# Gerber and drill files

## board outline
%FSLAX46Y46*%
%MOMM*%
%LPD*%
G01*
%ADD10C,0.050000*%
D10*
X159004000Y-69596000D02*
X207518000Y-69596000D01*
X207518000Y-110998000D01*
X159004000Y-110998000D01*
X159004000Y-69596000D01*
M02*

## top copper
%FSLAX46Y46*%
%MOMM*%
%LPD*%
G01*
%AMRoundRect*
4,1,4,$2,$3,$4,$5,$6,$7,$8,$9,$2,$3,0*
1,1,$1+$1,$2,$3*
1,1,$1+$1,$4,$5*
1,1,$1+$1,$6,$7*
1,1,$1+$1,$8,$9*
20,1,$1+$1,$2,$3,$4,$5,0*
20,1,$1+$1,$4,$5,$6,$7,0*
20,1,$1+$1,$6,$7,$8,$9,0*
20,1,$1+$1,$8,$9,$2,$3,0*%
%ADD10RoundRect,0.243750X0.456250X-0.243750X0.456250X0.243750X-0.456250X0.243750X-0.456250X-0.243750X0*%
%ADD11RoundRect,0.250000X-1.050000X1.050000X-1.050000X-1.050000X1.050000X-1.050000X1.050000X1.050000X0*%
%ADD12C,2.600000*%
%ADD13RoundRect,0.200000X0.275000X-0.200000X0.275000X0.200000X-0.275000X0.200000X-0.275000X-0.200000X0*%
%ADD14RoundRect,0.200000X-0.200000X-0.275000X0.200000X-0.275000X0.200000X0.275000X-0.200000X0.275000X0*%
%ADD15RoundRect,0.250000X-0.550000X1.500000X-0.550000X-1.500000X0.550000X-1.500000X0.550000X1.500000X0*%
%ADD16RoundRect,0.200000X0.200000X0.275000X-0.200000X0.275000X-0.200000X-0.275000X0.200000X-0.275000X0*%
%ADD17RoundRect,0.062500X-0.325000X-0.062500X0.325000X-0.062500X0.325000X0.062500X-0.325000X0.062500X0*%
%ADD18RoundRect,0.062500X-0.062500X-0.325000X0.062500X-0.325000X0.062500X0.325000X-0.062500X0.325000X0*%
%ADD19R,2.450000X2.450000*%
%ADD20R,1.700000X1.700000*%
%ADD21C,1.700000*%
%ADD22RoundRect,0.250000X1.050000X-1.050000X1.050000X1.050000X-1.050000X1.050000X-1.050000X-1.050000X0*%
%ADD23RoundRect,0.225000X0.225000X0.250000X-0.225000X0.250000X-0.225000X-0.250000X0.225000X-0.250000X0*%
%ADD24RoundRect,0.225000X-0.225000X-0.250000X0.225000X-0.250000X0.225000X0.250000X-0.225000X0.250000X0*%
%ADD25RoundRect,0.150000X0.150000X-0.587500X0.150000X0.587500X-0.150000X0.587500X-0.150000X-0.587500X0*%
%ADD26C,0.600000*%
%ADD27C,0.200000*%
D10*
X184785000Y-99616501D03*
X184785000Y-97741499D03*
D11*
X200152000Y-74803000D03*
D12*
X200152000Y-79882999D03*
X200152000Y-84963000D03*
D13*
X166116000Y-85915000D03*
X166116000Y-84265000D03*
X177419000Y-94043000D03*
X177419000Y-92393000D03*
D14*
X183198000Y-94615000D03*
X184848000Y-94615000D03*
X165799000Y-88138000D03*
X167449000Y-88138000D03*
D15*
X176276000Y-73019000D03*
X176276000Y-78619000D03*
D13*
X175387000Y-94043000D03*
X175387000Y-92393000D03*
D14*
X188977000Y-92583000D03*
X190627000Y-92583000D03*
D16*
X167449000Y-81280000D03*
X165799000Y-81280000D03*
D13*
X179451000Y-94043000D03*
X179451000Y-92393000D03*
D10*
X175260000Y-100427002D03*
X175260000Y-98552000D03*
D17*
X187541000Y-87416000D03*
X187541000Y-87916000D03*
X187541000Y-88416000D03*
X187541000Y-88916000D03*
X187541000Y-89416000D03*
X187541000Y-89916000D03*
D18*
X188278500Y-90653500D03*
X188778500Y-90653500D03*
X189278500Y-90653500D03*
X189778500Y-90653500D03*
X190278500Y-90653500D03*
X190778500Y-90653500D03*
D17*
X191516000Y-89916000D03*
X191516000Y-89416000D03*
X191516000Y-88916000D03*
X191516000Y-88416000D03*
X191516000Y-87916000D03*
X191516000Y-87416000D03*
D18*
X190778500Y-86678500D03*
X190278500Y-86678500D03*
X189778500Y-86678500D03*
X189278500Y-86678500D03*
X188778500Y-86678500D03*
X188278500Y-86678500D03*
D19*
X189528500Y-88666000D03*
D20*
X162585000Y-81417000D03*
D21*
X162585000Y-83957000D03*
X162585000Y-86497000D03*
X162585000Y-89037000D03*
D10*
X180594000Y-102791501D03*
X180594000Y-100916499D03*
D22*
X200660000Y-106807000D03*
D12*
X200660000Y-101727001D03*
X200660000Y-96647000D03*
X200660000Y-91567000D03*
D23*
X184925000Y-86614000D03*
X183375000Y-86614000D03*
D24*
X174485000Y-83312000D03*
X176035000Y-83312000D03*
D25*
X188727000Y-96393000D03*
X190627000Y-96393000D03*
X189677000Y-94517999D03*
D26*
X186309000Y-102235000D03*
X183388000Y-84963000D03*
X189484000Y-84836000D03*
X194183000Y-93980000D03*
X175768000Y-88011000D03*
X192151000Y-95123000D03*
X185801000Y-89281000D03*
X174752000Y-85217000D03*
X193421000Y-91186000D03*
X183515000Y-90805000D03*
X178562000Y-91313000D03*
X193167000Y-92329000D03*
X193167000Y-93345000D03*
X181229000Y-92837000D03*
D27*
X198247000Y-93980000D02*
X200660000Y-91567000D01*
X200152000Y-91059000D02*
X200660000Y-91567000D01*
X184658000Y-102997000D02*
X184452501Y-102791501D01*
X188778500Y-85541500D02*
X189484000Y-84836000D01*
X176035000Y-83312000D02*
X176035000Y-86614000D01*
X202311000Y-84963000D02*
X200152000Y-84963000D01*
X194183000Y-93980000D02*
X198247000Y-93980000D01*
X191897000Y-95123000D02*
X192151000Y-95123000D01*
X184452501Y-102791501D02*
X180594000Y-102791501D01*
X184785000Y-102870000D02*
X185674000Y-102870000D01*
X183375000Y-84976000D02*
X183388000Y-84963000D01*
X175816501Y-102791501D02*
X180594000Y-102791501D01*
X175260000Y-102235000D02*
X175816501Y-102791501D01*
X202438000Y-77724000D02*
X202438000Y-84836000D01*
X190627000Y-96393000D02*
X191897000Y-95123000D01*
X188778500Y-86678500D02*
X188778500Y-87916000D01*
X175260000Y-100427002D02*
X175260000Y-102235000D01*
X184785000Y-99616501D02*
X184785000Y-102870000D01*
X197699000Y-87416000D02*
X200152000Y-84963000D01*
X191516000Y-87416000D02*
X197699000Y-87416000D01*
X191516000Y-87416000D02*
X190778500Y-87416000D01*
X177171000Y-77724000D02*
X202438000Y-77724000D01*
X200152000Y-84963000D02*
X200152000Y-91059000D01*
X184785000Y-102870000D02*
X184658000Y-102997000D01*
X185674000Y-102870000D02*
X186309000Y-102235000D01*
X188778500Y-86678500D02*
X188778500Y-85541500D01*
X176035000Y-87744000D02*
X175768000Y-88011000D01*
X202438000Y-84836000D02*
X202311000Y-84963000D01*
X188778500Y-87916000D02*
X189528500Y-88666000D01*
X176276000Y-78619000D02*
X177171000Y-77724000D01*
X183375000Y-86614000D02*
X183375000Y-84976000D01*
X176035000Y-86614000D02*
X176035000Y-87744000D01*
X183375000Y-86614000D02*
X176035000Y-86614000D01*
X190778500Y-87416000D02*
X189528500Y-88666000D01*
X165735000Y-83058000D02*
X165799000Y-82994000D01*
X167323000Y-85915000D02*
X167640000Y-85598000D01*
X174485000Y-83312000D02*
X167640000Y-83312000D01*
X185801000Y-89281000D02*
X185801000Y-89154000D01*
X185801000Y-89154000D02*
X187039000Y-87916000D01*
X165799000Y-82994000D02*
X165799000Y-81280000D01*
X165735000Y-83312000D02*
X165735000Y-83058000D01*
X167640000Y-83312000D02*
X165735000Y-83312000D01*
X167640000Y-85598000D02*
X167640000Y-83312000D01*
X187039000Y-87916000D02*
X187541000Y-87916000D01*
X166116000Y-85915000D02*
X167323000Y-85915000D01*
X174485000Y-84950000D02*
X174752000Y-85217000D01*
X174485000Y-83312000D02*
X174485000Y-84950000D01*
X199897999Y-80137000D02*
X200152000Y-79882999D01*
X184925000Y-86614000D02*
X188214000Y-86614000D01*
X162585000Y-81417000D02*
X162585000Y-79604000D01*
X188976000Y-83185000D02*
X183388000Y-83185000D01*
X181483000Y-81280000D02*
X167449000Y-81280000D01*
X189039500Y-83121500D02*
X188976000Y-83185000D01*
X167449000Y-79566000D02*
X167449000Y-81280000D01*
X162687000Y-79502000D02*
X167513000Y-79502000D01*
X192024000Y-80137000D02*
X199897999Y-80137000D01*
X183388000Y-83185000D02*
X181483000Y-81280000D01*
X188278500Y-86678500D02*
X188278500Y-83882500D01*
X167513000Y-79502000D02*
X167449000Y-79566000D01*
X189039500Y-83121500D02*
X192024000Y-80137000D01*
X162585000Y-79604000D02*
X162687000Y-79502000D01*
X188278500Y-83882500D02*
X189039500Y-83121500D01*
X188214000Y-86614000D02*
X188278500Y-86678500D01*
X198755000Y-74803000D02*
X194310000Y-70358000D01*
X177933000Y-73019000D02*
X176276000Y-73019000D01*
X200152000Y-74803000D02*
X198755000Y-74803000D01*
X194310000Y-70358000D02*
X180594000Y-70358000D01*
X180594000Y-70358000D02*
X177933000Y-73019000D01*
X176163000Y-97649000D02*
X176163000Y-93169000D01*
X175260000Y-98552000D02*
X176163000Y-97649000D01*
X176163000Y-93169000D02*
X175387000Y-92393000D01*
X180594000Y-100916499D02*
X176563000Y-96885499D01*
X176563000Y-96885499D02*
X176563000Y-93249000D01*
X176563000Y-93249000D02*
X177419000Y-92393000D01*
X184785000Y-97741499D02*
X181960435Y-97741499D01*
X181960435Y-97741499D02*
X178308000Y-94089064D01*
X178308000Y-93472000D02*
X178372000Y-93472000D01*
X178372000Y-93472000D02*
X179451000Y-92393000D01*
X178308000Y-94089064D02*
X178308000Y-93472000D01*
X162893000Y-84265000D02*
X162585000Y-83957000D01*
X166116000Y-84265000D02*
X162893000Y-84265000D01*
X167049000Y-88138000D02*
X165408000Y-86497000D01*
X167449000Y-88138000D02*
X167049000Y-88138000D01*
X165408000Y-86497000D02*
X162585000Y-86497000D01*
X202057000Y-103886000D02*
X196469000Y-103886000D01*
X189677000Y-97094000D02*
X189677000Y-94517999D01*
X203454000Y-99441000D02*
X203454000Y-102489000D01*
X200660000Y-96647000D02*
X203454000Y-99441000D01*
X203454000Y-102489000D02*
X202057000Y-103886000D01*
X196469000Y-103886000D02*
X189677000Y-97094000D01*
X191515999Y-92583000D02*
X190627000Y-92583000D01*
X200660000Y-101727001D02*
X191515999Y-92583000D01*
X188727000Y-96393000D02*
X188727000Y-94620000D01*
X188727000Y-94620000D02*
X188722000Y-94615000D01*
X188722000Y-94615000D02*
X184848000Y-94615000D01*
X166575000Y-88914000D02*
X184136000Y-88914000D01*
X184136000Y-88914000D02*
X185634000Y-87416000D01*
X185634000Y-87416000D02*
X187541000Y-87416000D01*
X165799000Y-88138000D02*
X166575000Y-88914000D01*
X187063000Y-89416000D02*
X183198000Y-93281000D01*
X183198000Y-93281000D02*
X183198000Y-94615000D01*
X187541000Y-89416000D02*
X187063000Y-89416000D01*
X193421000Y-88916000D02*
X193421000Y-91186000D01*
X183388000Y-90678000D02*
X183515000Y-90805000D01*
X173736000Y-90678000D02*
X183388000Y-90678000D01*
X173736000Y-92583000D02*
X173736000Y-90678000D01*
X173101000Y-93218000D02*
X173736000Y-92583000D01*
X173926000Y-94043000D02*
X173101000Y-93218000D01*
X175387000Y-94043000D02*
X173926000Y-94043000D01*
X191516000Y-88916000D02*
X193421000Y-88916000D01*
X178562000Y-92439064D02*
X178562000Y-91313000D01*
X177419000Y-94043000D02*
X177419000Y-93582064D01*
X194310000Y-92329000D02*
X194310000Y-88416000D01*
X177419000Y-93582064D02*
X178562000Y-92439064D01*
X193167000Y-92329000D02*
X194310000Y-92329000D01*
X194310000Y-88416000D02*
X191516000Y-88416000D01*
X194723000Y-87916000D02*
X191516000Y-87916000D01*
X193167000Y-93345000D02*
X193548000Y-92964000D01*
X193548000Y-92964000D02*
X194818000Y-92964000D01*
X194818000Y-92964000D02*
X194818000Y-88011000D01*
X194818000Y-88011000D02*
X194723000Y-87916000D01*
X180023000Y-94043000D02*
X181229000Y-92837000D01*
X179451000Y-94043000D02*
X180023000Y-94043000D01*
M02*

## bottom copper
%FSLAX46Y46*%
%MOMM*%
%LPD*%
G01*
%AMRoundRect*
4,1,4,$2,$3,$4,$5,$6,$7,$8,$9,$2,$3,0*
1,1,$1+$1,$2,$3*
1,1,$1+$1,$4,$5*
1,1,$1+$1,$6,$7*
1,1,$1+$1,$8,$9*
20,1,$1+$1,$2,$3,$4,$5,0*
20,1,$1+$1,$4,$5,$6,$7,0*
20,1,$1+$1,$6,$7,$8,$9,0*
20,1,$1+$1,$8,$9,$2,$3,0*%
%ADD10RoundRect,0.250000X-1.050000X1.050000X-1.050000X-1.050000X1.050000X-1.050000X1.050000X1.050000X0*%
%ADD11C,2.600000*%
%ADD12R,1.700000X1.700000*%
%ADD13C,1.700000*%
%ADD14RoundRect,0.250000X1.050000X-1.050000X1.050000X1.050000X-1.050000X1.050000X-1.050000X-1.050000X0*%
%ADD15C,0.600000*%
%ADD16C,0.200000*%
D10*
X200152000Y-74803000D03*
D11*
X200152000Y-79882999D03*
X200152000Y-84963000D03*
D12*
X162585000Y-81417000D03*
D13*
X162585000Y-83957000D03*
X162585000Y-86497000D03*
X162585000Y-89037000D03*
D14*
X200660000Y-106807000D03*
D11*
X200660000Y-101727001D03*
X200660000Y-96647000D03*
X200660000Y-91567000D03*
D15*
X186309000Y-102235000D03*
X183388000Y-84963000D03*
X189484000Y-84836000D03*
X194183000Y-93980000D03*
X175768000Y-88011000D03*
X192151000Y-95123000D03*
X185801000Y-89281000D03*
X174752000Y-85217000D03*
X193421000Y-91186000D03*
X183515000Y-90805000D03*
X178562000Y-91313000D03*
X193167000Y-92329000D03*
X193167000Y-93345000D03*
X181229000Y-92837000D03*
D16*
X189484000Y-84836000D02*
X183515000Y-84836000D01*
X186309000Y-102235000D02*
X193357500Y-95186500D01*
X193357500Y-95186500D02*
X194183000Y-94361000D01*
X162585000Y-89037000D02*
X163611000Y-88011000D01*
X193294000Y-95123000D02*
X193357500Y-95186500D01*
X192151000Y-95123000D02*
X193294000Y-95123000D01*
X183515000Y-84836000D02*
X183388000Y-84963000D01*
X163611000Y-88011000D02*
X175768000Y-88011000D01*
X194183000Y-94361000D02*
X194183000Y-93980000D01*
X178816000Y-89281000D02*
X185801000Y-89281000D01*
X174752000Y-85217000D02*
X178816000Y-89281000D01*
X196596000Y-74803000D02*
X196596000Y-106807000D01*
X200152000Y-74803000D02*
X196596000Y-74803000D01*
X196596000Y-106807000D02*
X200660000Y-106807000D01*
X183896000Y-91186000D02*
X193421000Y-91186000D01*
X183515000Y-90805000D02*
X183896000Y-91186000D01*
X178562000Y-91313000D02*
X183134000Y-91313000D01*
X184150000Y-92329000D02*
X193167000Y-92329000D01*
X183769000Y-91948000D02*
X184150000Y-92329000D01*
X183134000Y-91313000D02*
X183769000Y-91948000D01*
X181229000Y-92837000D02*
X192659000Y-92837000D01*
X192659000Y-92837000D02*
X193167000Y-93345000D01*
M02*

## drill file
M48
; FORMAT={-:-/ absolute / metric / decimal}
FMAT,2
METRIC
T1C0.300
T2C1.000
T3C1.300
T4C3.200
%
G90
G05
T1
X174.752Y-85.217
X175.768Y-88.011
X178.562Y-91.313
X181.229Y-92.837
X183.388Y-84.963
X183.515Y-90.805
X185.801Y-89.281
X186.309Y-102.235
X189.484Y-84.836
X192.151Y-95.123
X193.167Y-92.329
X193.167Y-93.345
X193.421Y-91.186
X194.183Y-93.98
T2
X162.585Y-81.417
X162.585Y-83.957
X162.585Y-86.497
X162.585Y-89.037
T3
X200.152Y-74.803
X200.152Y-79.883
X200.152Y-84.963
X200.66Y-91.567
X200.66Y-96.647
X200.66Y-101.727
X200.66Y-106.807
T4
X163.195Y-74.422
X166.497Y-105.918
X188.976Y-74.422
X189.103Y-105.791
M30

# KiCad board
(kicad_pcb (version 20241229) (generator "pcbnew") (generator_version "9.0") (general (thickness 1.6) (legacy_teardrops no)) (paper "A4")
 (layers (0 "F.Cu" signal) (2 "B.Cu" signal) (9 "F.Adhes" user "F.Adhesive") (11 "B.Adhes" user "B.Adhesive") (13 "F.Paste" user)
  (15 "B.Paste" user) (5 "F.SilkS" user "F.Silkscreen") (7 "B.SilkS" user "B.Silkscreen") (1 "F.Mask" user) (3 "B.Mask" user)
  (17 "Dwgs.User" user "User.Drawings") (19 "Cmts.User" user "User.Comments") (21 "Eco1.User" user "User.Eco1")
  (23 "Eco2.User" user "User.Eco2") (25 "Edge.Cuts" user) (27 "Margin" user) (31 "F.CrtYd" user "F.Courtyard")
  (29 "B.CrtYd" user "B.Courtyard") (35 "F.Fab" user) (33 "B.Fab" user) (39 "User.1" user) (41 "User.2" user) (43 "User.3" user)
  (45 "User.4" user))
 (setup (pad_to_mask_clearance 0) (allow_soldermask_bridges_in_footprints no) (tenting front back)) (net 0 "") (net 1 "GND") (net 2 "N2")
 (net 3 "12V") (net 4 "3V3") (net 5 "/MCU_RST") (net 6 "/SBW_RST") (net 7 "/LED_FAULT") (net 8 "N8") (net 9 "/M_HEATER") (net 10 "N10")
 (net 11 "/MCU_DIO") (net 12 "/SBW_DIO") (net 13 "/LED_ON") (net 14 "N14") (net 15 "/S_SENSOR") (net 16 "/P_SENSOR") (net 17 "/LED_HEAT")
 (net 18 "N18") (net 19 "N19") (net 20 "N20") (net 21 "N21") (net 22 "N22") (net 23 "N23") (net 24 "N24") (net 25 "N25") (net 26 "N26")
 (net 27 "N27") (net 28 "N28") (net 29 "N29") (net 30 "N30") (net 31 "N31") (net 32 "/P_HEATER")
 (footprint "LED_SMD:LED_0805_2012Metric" (layer "F.Cu") (at 184.785 98.679 90)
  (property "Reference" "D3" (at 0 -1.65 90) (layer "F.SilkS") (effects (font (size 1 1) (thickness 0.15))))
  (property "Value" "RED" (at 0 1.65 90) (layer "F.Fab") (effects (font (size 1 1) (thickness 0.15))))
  (pad "1" smd roundrect (at -0.937501 0 90) (size 0.975 1.4) (layers "F.Cu" "F.Mask" "F.Paste") (roundrect_rratio 0.25) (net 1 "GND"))
  (pad "2" smd roundrect (at 0.937501 0 90) (size 0.975 1.4) (layers "F.Cu" "F.Mask" "F.Paste") (roundrect_rratio 0.25) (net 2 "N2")))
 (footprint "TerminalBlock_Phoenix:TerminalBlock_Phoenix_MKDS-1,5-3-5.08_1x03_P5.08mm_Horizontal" (layer "F.Cu") (at 200.152 74.803 -90)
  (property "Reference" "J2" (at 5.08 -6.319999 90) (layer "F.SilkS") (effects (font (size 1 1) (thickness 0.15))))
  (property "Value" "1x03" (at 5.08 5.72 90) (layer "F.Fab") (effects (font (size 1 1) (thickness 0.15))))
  (pad "1" thru_hole roundrect (at 0 0 270) (size 2.6 2.6) (drill 1.3) (layers "*.Cu" "*.Mask") (remove_unused_layers no)
   (roundrect_rratio 0.096154) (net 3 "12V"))
  (pad "2" thru_hole circle (at 5.079999 0 270) (size 2.6 2.6) (drill 1.3) (layers "*.Cu" "*.Mask") (remove_unused_layers no) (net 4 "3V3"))
  (pad "3" thru_hole circle (at 10.16 0 270) (size 2.6 2.6) (drill 1.3) (layers "*.Cu" "*.Mask") (remove_unused_layers no) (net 1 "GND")))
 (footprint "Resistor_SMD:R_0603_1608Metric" (layer "F.Cu") (at 166.116 85.09 90)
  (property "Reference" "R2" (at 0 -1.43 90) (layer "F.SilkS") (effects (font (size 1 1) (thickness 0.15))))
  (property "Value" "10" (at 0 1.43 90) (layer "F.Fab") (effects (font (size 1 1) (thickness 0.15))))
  (pad "1" smd roundrect (at -0.825 0 90) (size 0.8 0.95) (layers "F.Cu" "F.Mask" "F.Paste") (roundrect_rratio 0.25) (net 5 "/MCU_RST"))
  (pad "2" smd roundrect (at 0.825 0 90) (size 0.8 0.95) (layers "F.Cu" "F.Mask" "F.Paste") (roundrect_rratio 0.25) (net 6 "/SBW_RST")))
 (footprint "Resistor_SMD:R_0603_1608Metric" (layer "F.Cu") (at 177.419 93.218 90)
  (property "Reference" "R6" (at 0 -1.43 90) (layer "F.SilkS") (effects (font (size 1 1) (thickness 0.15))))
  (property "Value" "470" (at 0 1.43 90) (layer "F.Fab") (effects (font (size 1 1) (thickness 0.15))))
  (pad "1" smd roundrect (at -0.825 0 90) (size 0.8 0.95) (layers "F.Cu" "F.Mask" "F.Paste") (roundrect_rratio 0.25) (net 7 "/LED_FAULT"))
  (pad "2" smd roundrect (at 0.825 0 90) (size 0.8 0.95) (layers "F.Cu" "F.Mask" "F.Paste") (roundrect_rratio 0.25) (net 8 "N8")))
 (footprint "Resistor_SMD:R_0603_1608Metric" (layer "F.Cu") (at 184.023 94.615)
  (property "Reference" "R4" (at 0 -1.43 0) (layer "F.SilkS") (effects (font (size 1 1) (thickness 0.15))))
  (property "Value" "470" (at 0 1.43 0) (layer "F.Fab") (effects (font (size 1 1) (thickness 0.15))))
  (pad "1" smd roundrect (at -0.825 0) (size 0.8 0.95) (layers "F.Cu" "F.Mask" "F.Paste") (roundrect_rratio 0.25) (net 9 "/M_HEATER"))
  (pad "2" smd roundrect (at 0.825 0) (size 0.8 0.95) (layers "F.Cu" "F.Mask" "F.Paste") (roundrect_rratio 0.25) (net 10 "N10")))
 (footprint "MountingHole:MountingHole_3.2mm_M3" (layer "F.Cu") (at 163.195 74.422)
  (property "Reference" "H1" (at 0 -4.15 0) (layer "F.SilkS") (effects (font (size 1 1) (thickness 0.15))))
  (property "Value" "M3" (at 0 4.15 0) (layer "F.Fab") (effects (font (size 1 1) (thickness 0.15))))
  (pad "" np_thru_hole circle (at 0 0) (size 3.2 3.2) (drill 3.2) (layers "*.Cu" "*.Mask")))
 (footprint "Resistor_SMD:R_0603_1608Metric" (layer "F.Cu") (at 166.624 88.138)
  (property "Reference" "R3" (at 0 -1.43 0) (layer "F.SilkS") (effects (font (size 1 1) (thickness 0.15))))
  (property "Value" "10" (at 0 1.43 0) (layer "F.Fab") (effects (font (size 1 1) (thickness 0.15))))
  (pad "1" smd roundrect (at -0.825 0) (size 0.8 0.95) (layers "F.Cu" "F.Mask" "F.Paste") (roundrect_rratio 0.25) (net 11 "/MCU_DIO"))
  (pad "2" smd roundrect (at 0.825 0) (size 0.8 0.95) (layers "F.Cu" "F.Mask" "F.Paste") (roundrect_rratio 0.25) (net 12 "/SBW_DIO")))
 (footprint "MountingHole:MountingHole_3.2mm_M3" (layer "F.Cu") (at 189.103 105.791)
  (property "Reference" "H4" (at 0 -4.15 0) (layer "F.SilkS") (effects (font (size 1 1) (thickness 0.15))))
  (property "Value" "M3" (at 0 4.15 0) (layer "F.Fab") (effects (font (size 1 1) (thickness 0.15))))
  (pad "" np_thru_hole circle (at 0 0) (size 3.2 3.2) (drill 3.2) (layers "*.Cu" "*.Mask")))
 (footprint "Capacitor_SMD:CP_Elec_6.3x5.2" (layer "F.Cu") (at 176.276 75.819 -90)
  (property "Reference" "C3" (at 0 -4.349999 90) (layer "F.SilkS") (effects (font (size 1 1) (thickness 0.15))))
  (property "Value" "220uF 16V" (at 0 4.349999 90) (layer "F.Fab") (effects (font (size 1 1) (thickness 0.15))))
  (pad "1" smd roundrect (at -2.8 0 270) (size 3.5 1.6) (layers "F.Cu" "F.Mask" "F.Paste") (roundrect_rratio 0.15625) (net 3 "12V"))
  (pad "2" smd roundrect (at 2.8 0 270) (size 3.5 1.6) (layers "F.Cu" "F.Mask" "F.Paste") (roundrect_rratio 0.15625) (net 1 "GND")))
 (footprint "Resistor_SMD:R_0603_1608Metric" (layer "F.Cu") (at 175.387 93.218 90)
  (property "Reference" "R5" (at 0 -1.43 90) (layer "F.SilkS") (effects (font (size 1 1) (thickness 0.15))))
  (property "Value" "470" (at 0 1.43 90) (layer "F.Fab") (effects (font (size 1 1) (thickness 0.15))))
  (pad "1" smd roundrect (at -0.825 0 90) (size 0.8 0.95) (layers "F.Cu" "F.Mask" "F.Paste") (roundrect_rratio 0.25) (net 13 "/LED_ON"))
  (pad "2" smd roundrect (at 0.825 0 90) (size 0.8 0.95) (layers "F.Cu" "F.Mask" "F.Paste") (roundrect_rratio 0.25) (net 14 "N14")))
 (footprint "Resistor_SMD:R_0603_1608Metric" (layer "F.Cu") (at 189.802 92.583)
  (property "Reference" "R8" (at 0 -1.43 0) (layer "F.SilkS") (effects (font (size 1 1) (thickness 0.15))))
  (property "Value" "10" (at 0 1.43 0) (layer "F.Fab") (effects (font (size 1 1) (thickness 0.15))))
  (pad "1" smd roundrect (at -0.825 0) (size 0.8 0.95) (layers "F.Cu" "F.Mask" "F.Paste") (roundrect_rratio 0.25) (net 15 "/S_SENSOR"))
  (pad "2" smd roundrect (at 0.825 0) (size 0.8 0.95) (layers "F.Cu" "F.Mask" "F.Paste") (roundrect_rratio 0.25) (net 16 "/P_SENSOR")))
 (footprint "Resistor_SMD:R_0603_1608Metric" (layer "F.Cu") (at 166.624 81.28 180)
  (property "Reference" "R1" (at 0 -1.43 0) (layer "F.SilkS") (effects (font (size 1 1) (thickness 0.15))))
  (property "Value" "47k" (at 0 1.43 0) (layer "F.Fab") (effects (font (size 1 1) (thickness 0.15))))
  (pad "1" smd roundrect (at -0.825 0 180) (size 0.8 0.95) (layers "F.Cu" "F.Mask" "F.Paste") (roundrect_rratio 0.25) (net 4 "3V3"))
  (pad "2" smd roundrect (at 0.825 0 180) (size 0.8 0.95) (layers "F.Cu" "F.Mask" "F.Paste") (roundrect_rratio 0.25) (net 5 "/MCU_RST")))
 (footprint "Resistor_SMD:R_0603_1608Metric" (layer "F.Cu") (at 179.451 93.218 90)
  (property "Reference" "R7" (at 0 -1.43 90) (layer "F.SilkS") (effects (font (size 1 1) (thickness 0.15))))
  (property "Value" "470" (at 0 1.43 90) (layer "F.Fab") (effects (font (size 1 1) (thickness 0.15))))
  (pad "1" smd roundrect (at -0.825 0 90) (size 0.8 0.95) (layers "F.Cu" "F.Mask" "F.Paste") (roundrect_rratio 0.25) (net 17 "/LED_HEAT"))
  (pad "2" smd roundrect (at 0.825 0 90) (size 0.8 0.95) (layers "F.Cu" "F.Mask" "F.Paste") (roundrect_rratio 0.25) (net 2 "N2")))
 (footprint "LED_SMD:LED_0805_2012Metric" (layer "F.Cu") (at 175.26 99.489501 90)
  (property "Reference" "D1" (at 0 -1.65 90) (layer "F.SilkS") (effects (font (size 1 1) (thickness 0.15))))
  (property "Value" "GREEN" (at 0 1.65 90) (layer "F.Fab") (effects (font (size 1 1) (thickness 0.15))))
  (pad "1" smd roundrect (at -0.937501 0 90) (size 0.975 1.4) (layers "F.Cu" "F.Mask" "F.Paste") (roundrect_rratio 0.25) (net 1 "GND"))
  (pad "2" smd roundrect (at 0.937501 0 90) (size 0.975 1.4) (layers "F.Cu" "F.Mask" "F.Paste") (roundrect_rratio 0.25) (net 14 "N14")))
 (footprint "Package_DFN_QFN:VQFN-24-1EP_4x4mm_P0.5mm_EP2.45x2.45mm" (layer "F.Cu") (at 189.5285 88.666)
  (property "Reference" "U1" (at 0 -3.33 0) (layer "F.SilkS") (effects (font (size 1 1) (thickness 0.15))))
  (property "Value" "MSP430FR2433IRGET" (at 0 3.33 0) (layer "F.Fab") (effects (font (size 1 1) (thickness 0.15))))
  (pad "" smd roundrect (at -0.82 -0.82) (size 0.66 0.66) (layers "F.Paste") (roundrect_rratio 0.25))
  (pad "" smd roundrect (at -0.82 0) (size 0.66 0.66) (layers "F.Paste") (roundrect_rratio 0.25))
  (pad "" smd roundrect (at -0.82 0.82) (size 0.66 0.66) (layers "F.Paste") (roundrect_rratio 0.25))
  (pad "" smd roundrect (at 0 -0.82) (size 0.66 0.66) (layers "F.Paste") (roundrect_rratio 0.25))
  (pad "" smd roundrect (at 0 0) (size 0.66 0.66) (layers "F.Paste") (roundrect_rratio 0.25))
  (pad "" smd roundrect (at 0 0.82) (size 0.66 0.66) (layers "F.Paste") (roundrect_rratio 0.25))
  (pad "" smd roundrect (at 0.82 -0.82) (size 0.66 0.66) (layers "F.Paste") (roundrect_rratio 0.25))
  (pad "" smd roundrect (at 0.82 0) (size 0.66 0.66) (layers "F.Paste") (roundrect_rratio 0.25))
  (pad "" smd roundrect (at 0.82 0.82) (size 0.66 0.66) (layers "F.Paste") (roundrect_rratio 0.25))
  (pad "1" smd roundrect (at -1.9875 -1.25) (size 0.775 0.25) (layers "F.Cu" "F.Mask" "F.Paste") (roundrect_rratio 0.25) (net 11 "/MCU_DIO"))
  (pad "2" smd roundrect (at -1.9875 -0.75) (size 0.775 0.25) (layers "F.Cu" "F.Mask" "F.Paste") (roundrect_rratio 0.25) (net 5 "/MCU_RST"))
  (pad "3" smd roundrect (at -1.9875 -0.25) (size 0.775 0.25) (layers "F.Cu" "F.Mask" "F.Paste") (roundrect_rratio 0.25) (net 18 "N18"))
  (pad "4" smd roundrect (at -1.9875 0.25) (size 0.775 0.25) (layers "F.Cu" "F.Mask" "F.Paste") (roundrect_rratio 0.25) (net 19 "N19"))
  (pad "5" smd roundrect (at -1.9875 0.75) (size 0.775 0.25) (layers "F.Cu" "F.Mask" "F.Paste") (roundrect_rratio 0.25) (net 9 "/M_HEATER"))
  (pad "6" smd roundrect (at -1.9875 1.25) (size 0.775 0.25) (layers "F.Cu" "F.Mask" "F.Paste") (roundrect_rratio 0.25) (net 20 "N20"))
  (pad "7" smd roundrect (at -1.25 1.9875) (size 0.25 0.775) (layers "F.Cu" "F.Mask" "F.Paste") (roundrect_rratio 0.25) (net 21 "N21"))
  (pad "8" smd roundrect (at -0.75 1.9875) (size 0.25 0.775) (layers "F.Cu" "F.Mask" "F.Paste") (roundrect_rratio 0.25) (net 15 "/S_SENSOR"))
  (pad "9" smd roundrect (at -0.25 1.9875) (size 0.25 0.775) (layers "F.Cu" "F.Mask" "F.Paste") (roundrect_rratio 0.25) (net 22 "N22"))
  (pad "10" smd roundrect (at 0.25 1.9875) (size 0.25 0.775) (layers "F.Cu" "F.Mask" "F.Paste") (roundrect_rratio 0.25) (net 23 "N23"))
  (pad "11" smd roundrect (at 0.75 1.9875) (size 0.25 0.775) (layers "F.Cu" "F.Mask" "F.Paste") (roundrect_rratio 0.25) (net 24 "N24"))
  (pad "12" smd roundrect (at 1.25 1.9875) (size 0.25 0.775) (layers "F.Cu" "F.Mask" "F.Paste") (roundrect_rratio 0.25) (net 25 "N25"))
  (pad "13" smd roundrect (at 1.9875 1.25) (size 0.775 0.25) (layers "F.Cu" "F.Mask" "F.Paste") (roundrect_rratio 0.25) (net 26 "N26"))
  (pad "14" smd roundrect (at 1.9875 0.75) (size 0.775 0.25) (layers "F.Cu" "F.Mask" "F.Paste") (roundrect_rratio 0.25) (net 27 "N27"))
  (pad "15" smd roundrect (at 1.9875 0.25) (size 0.775 0.25) (layers "F.Cu" "F.Mask" "F.Paste") (roundrect_rratio 0.25) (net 13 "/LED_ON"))
  (pad "16" smd roundrect (at 1.9875 -0.25) (size 0.775 0.25) (layers "F.Cu" "F.Mask" "F.Paste") (roundrect_rratio 0.25)
   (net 7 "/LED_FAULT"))
  (pad "17" smd roundrect (at 1.9875 -0.75) (size 0.775 0.25) (layers "F.Cu" "F.Mask" "F.Paste") (roundrect_rratio 0.25)
   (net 17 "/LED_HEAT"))
  (pad "18" smd roundrect (at 1.9875 -1.25) (size 0.775 0.25) (layers "F.Cu" "F.Mask" "F.Paste") (roundrect_rratio 0.25) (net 1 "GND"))
  (pad "19" smd roundrect (at 1.25 -1.9875) (size 0.25 0.775) (layers "F.Cu" "F.Mask" "F.Paste") (roundrect_rratio 0.25) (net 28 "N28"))
  (pad "20" smd roundrect (at 0.75 -1.9875) (size 0.25 0.775) (layers "F.Cu" "F.Mask" "F.Paste") (roundrect_rratio 0.25) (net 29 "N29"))
  (pad "21" smd roundrect (at 0.25 -1.9875) (size 0.25 0.775) (layers "F.Cu" "F.Mask" "F.Paste") (roundrect_rratio 0.25) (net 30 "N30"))
  (pad "22" smd roundrect (at -0.25 -1.9875) (size 0.25 0.775) (layers "F.Cu" "F.Mask" "F.Paste") (roundrect_rratio 0.25) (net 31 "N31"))
  (pad "23" smd roundrect (at -0.75 -1.9875) (size 0.25 0.775) (layers "F.Cu" "F.Mask" "F.Paste") (roundrect_rratio 0.25) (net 1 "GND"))
  (pad "24" smd roundrect (at -1.25 -1.9875) (size 0.25 0.775) (layers "F.Cu" "F.Mask" "F.Paste") (roundrect_rratio 0.25) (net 4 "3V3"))
  (pad "25" smd rect (at 0 0) (size 2.45 2.45) (layers "F.Cu" "F.Mask") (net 1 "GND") (zone_connect 2)))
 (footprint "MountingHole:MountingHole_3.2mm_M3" (layer "F.Cu") (at 166.497 105.918)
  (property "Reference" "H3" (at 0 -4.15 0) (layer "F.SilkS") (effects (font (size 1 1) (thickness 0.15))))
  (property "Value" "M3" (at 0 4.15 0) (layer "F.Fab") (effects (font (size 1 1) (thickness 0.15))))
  (pad "" np_thru_hole circle (at 0 0) (size 3.2 3.2) (drill 3.2) (layers "*.Cu" "*.Mask")))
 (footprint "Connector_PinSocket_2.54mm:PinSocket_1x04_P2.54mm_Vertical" (layer "F.Cu") (at 162.585 81.417)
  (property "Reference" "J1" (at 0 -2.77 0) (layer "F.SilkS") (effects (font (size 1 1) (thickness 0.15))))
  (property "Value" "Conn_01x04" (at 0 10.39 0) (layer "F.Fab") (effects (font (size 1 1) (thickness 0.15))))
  (pad "1" thru_hole rect (at 0 0) (size 1.7 1.7) (drill 1) (layers "*.Cu" "*.Mask") (remove_unused_layers no) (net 4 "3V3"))
  (pad "2" thru_hole circle (at 0 2.54) (size 1.7 1.7) (drill 1) (layers "*.Cu" "*.Mask") (remove_unused_layers no) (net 6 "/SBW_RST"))
  (pad "3" thru_hole circle (at 0 5.08) (size 1.7 1.7) (drill 1) (layers "*.Cu" "*.Mask") (remove_unused_layers no) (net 12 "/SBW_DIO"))
  (pad "4" thru_hole circle (at 0 7.62) (size 1.7 1.7) (drill 1) (layers "*.Cu" "*.Mask") (remove_unused_layers no) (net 1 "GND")))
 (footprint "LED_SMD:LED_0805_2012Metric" (layer "F.Cu") (at 180.594 101.854 90)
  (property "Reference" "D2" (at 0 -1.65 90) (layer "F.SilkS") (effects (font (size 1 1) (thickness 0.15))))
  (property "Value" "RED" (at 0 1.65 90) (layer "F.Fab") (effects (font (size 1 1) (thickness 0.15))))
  (pad "1" smd roundrect (at -0.937501 0 90) (size 0.975 1.4) (layers "F.Cu" "F.Mask" "F.Paste") (roundrect_rratio 0.25) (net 1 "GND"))
  (pad "2" smd roundrect (at 0.937501 0 90) (size 0.975 1.4) (layers "F.Cu" "F.Mask" "F.Paste") (roundrect_rratio 0.25) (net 8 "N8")))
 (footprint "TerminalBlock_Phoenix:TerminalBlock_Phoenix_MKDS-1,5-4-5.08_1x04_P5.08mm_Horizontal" (layer "F.Cu") (at 200.66 106.807 90)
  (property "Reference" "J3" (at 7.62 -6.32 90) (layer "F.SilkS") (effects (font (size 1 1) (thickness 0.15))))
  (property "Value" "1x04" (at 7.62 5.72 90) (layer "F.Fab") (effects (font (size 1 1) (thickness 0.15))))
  (pad "1" thru_hole roundrect (at 0 0 90) (size 2.6 2.6) (drill 1.3) (layers "*.Cu" "*.Mask") (remove_unused_layers no)
   (roundrect_rratio 0.096154) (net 3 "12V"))
  (pad "2" thru_hole circle (at 5.079999 0 90) (size 2.6 2.6) (drill 1.3) (layers "*.Cu" "*.Mask") (remove_unused_layers no)
   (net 16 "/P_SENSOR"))
  (pad "3" thru_hole circle (at 10.16 0 90) (size 2.6 2.6) (drill 1.3) (layers "*.Cu" "*.Mask") (remove_unused_layers no)
   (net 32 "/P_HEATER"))
  (pad "4" thru_hole circle (at 15.24 0 90) (size 2.6 2.6) (drill 1.3) (layers "*.Cu" "*.Mask") (remove_unused_layers no) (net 1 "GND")))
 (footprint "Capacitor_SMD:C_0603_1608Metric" (layer "F.Cu") (at 184.15 86.614 180)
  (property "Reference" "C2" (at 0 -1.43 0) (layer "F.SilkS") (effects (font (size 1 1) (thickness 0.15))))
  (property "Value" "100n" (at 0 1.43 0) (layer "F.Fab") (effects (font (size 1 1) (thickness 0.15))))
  (pad "1" smd roundrect (at -0.775 0 180) (size 0.9 0.95) (layers "F.Cu" "F.Mask" "F.Paste") (roundrect_rratio 0.25) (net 4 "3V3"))
  (pad "2" smd roundrect (at 0.775 0 180) (size 0.9 0.95) (layers "F.Cu" "F.Mask" "F.Paste") (roundrect_rratio 0.25) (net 1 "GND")))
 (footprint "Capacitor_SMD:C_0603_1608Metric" (layer "F.Cu") (at 175.26 83.312)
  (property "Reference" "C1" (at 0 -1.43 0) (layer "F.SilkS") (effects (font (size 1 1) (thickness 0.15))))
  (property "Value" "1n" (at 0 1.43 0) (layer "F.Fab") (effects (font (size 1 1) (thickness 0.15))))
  (pad "1" smd roundrect (at -0.775 0) (size 0.9 0.95) (layers "F.Cu" "F.Mask" "F.Paste") (roundrect_rratio 0.25) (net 5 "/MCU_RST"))
  (pad "2" smd roundrect (at 0.775 0) (size 0.9 0.95) (layers "F.Cu" "F.Mask" "F.Paste") (roundrect_rratio 0.25) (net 1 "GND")))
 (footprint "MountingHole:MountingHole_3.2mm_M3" (layer "F.Cu") (at 188.976 74.422)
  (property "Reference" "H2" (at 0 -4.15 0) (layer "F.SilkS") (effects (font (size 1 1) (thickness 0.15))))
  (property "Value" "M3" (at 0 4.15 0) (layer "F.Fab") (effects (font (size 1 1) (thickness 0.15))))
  (pad "" np_thru_hole circle (at 0 0) (size 3.2 3.2) (drill 3.2) (layers "*.Cu" "*.Mask")))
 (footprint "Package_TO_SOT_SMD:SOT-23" (layer "F.Cu") (at 189.677 95.4555 90)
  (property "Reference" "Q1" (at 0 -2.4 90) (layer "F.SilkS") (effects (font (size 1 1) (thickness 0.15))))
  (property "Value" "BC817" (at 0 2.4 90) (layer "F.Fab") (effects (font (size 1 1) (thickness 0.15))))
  (pad "1" smd roundrect (at -0.9375 -0.95 90) (size 1.475 0.6) (layers "F.Cu" "F.Mask" "F.Paste") (roundrect_rratio 0.25) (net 10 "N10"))
  (pad "2" smd roundrect (at -0.9375 0.95 90) (size 1.475 0.6) (layers "F.Cu" "F.Mask" "F.Paste") (roundrect_rratio 0.25) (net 1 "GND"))
  (pad "3" smd roundrect (at 0.937501 0 90) (size 1.475 0.6) (layers "F.Cu" "F.Mask" "F.Paste") (roundrect_rratio 0.25) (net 32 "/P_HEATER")))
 (gr_rect (start 159.004 69.596) (end 207.518 110.998) (stroke (width 0.05) (type default)) (fill no) (layer "Edge.Cuts"))
 (segment (start 198.247 93.98) (end 200.66 91.567) (width 0.2) (layer "F.Cu") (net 1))
 (segment (start 200.152 91.059) (end 200.66 91.567) (width 0.2) (layer "F.Cu") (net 1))
 (segment (start 184.658 102.997) (end 184.452501 102.791501) (width 0.2) (layer "F.Cu") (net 1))
 (segment (start 188.7785 85.5415) (end 189.484 84.836) (width 0.2) (layer "F.Cu") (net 1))
 (segment (start 176.035 83.312) (end 176.035 86.614) (width 0.2) (layer "F.Cu") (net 1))
 (segment (start 202.311 84.963) (end 200.152 84.963) (width 0.2) (layer "F.Cu") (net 1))
 (segment (start 194.183 93.98) (end 198.247 93.98) (width 0.2) (layer "F.Cu") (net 1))
 (segment (start 191.897 95.123) (end 192.151 95.123) (width 0.2) (layer "F.Cu") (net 1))
 (segment (start 184.452501 102.791501) (end 180.594 102.791501) (width 0.2) (layer "F.Cu") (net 1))
 (segment (start 184.785 102.87) (end 185.674 102.87) (width 0.2) (layer "F.Cu") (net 1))
 (segment (start 183.375 84.976) (end 183.388 84.963) (width 0.2) (layer "F.Cu") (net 1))
 (segment (start 175.816501 102.791501) (end 180.594 102.791501) (width 0.2) (layer "F.Cu") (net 1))
 (segment (start 175.26 102.235) (end 175.816501 102.791501) (width 0.2) (layer "F.Cu") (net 1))
 (segment (start 202.438 77.724) (end 202.438 84.836) (width 0.2) (layer "F.Cu") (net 1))
 (segment (start 190.627 96.393) (end 191.897 95.123) (width 0.2) (layer "F.Cu") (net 1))
 (segment (start 188.7785 86.6785) (end 188.7785 87.916) (width 0.2) (layer "F.Cu") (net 1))
 (segment (start 175.26 100.427002) (end 175.26 102.235) (width 0.2) (layer "F.Cu") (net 1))
 (segment (start 184.785 99.616501) (end 184.785 102.87) (width 0.2) (layer "F.Cu") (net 1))
 (segment (start 197.699 87.416) (end 200.152 84.963) (width 0.2) (layer "F.Cu") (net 1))
 (segment (start 191.516 87.416) (end 197.699 87.416) (width 0.2) (layer "F.Cu") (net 1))
 (segment (start 191.516 87.416) (end 190.7785 87.416) (width 0.2) (layer "F.Cu") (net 1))
 (segment (start 177.171 77.724) (end 202.438 77.724) (width 0.2) (layer "F.Cu") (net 1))
 (segment (start 200.152 84.963) (end 200.152 91.059) (width 0.2) (layer "F.Cu") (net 1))
 (segment (start 184.785 102.87) (end 184.658 102.997) (width 0.2) (layer "F.Cu") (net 1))
 (segment (start 185.674 102.87) (end 186.309 102.235) (width 0.2) (layer "F.Cu") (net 1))
 (segment (start 188.7785 86.6785) (end 188.7785 85.5415) (width 0.2) (layer "F.Cu") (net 1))
 (segment (start 176.035 87.744) (end 175.768 88.011) (width 0.2) (layer "F.Cu") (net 1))
 (segment (start 202.438 84.836) (end 202.311 84.963) (width 0.2) (layer "F.Cu") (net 1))
 (segment (start 188.7785 87.916) (end 189.5285 88.666) (width 0.2) (layer "F.Cu") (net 1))
 (segment (start 176.276 78.619) (end 177.171 77.724) (width 0.2) (layer "F.Cu") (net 1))
 (segment (start 183.375 86.614) (end 183.375 84.976) (width 0.2) (layer "F.Cu") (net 1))
 (segment (start 176.035 86.614) (end 176.035 87.744) (width 0.2) (layer "F.Cu") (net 1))
 (segment (start 183.375 86.614) (end 176.035 86.614) (width 0.2) (layer "F.Cu") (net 1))
 (segment (start 190.7785 87.416) (end 189.5285 88.666) (width 0.2) (layer "F.Cu") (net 1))
 (via (at 186.309 102.235) (size 0.6) (drill 0.3) (layers "F.Cu" "B.Cu") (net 1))
 (via (at 183.388 84.963) (size 0.6) (drill 0.3) (layers "F.Cu" "B.Cu") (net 1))
 (via (at 189.484 84.836) (size 0.6) (drill 0.3) (layers "F.Cu" "B.Cu") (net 1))
 (via (at 194.183 93.98) (size 0.6) (drill 0.3) (layers "F.Cu" "B.Cu") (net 1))
 (via (at 175.768 88.011) (size 0.6) (drill 0.3) (layers "F.Cu" "B.Cu") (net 1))
 (via (at 192.151 95.123) (size 0.6) (drill 0.3) (layers "F.Cu" "B.Cu") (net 1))
 (segment (start 189.484 84.836) (end 183.515 84.836) (width 0.2) (layer "B.Cu") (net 1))
 (segment (start 186.309 102.235) (end 193.3575 95.1865) (width 0.2) (layer "B.Cu") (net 1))
 (segment (start 193.3575 95.1865) (end 194.183 94.361) (width 0.2) (layer "B.Cu") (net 1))
 (segment (start 162.585 89.037) (end 163.611 88.011) (width 0.2) (layer "B.Cu") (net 1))
 (segment (start 193.294 95.123) (end 193.3575 95.1865) (width 0.2) (layer "B.Cu") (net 1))
 (segment (start 192.151 95.123) (end 193.294 95.123) (width 0.2) (layer "B.Cu") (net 1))
 (segment (start 183.515 84.836) (end 183.388 84.963) (width 0.2) (layer "B.Cu") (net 1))
 (segment (start 163.611 88.011) (end 175.768 88.011) (width 0.2) (layer "B.Cu") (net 1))
 (segment (start 194.183 94.361) (end 194.183 93.98) (width 0.2) (layer "B.Cu") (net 1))
 (segment (start 165.735 83.058) (end 165.799 82.994) (width 0.2) (layer "F.Cu") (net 5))
 (segment (start 167.323 85.915) (end 167.64 85.598) (width 0.2) (layer "F.Cu") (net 5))
 (segment (start 174.485 83.312) (end 167.64 83.312) (width 0.2) (layer "F.Cu") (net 5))
 (segment (start 185.801 89.281) (end 185.801 89.154) (width 0.2) (layer "F.Cu") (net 5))
 (segment (start 185.801 89.154) (end 187.039 87.916) (width 0.2) (layer "F.Cu") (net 5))
 (segment (start 165.799 82.994) (end 165.799 81.28) (width 0.2) (layer "F.Cu") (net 5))
 (segment (start 165.735 83.312) (end 165.735 83.058) (width 0.2) (layer "F.Cu") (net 5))
 (segment (start 167.64 83.312) (end 165.735 83.312) (width 0.2) (layer "F.Cu") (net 5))
 (segment (start 167.64 85.598) (end 167.64 83.312) (width 0.2) (layer "F.Cu") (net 5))
 (segment (start 187.039 87.916) (end 187.541 87.916) (width 0.2) (layer "F.Cu") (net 5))
 (segment (start 166.116 85.915) (end 167.323 85.915) (width 0.2) (layer "F.Cu") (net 5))
 (segment (start 174.485 84.95) (end 174.752 85.217) (width 0.2) (layer "F.Cu") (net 5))
 (segment (start 174.485 83.312) (end 174.485 84.95) (width 0.2) (layer "F.Cu") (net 5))
 (via (at 185.801 89.281) (size 0.6) (drill 0.3) (layers "F.Cu" "B.Cu") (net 5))
 (via (at 174.752 85.217) (size 0.6) (drill 0.3) (layers "F.Cu" "B.Cu") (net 5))
 (segment (start 178.816 89.281) (end 185.801 89.281) (width 0.2) (layer "B.Cu") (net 5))
 (segment (start 174.752 85.217) (end 178.816 89.281) (width 0.2) (layer "B.Cu") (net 5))
 (segment (start 199.897999 80.137) (end 200.152 79.882999) (width 0.2) (layer "F.Cu") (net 4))
 (segment (start 184.925 86.614) (end 188.214 86.614) (width 0.2) (layer "F.Cu") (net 4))
 (segment (start 162.585 81.417) (end 162.585 79.604) (width 0.2) (layer "F.Cu") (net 4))
 (segment (start 188.976 83.185) (end 183.388 83.185) (width 0.2) (layer "F.Cu") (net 4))
 (segment (start 181.483 81.28) (end 167.449 81.28) (width 0.2) (layer "F.Cu") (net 4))
 (segment (start 189.0395 83.1215) (end 188.976 83.185) (width 0.2) (layer "F.Cu") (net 4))
 (segment (start 167.449 79.566) (end 167.449 81.28) (width 0.2) (layer "F.Cu") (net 4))
 (segment (start 162.687 79.502) (end 167.513 79.502) (width 0.2) (layer "F.Cu") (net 4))
 (segment (start 192.024 80.137) (end 199.897999 80.137) (width 0.2) (layer "F.Cu") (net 4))
 (segment (start 183.388 83.185) (end 181.483 81.28) (width 0.2) (layer "F.Cu") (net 4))
 (segment (start 188.2785 86.6785) (end 188.2785 83.8825) (width 0.2) (layer "F.Cu") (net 4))
 (segment (start 167.513 79.502) (end 167.449 79.566) (width 0.2) (layer "F.Cu") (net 4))
 (segment (start 189.0395 83.1215) (end 192.024 80.137) (width 0.2) (layer "F.Cu") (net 4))
 (segment (start 162.585 79.604) (end 162.687 79.502) (width 0.2) (layer "F.Cu") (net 4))
 (segment (start 188.2785 83.8825) (end 189.0395 83.1215) (width 0.2) (layer "F.Cu") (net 4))
 (segment (start 188.214 86.614) (end 188.2785 86.6785) (width 0.2) (layer "F.Cu") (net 4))
 (segment (start 198.755 74.803) (end 194.31 70.358) (width 0.2) (layer "F.Cu") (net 3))
 (segment (start 177.933 73.019) (end 176.276 73.019) (width 0.2) (layer "F.Cu") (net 3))
 (segment (start 200.152 74.803) (end 198.755 74.803) (width 0.2) (layer "F.Cu") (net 3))
 (segment (start 194.31 70.358) (end 180.594 70.358) (width 0.2) (layer "F.Cu") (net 3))
 (segment (start 180.594 70.358) (end 177.933 73.019) (width 0.2) (layer "F.Cu") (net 3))
 (segment (start 196.596 74.803) (end 196.596 106.807) (width 0.2) (layer "B.Cu") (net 3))
 (segment (start 200.152 74.803) (end 196.596 74.803) (width 0.2) (layer "B.Cu") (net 3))
 (segment (start 196.596 106.807) (end 200.66 106.807) (width 0.2) (layer "B.Cu") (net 3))
 (segment (start 176.163 97.649) (end 176.163 93.169) (width 0.2) (layer "F.Cu") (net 14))
 (segment (start 175.26 98.552) (end 176.163 97.649) (width 0.2) (layer "F.Cu") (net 14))
 (segment (start 176.163 93.169) (end 175.387 92.393) (width 0.2) (layer "F.Cu") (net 14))
 (segment (start 180.594 100.916499) (end 176.563 96.885499) (width 0.2) (layer "F.Cu") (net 8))
 (segment (start 176.563 96.885499) (end 176.563 93.249) (width 0.2) (layer "F.Cu") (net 8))
 (segment (start 176.563 93.249) (end 177.419 92.393) (width 0.2) (layer "F.Cu") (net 8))
 (segment (start 184.785 97.741499) (end 181.960435 97.741499) (width 0.2) (layer "F.Cu") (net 2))
 (segment (start 181.960435 97.741499) (end 178.308 94.089064) (width 0.2) (layer "F.Cu") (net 2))
 (segment (start 178.308 93.472) (end 178.372 93.472) (width 0.2) (layer "F.Cu") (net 2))
 (segment (start 178.372 93.472) (end 179.451 92.393) (width 0.2) (layer "F.Cu") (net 2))
 (segment (start 178.308 94.089064) (end 178.308 93.472) (width 0.2) (layer "F.Cu") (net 2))
 (segment (start 162.893 84.265) (end 162.585 83.957) (width 0.2) (layer "F.Cu") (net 6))
 (segment (start 166.116 84.265) (end 162.893 84.265) (width 0.2) (layer "F.Cu") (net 6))
 (segment (start 167.049 88.138) (end 165.408 86.497) (width 0.2) (layer "F.Cu") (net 12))
 (segment (start 167.449 88.138) (end 167.049 88.138) (width 0.2) (layer "F.Cu") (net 12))
 (segment (start 165.408 86.497) (end 162.585 86.497) (width 0.2) (layer "F.Cu") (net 12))
 (segment (start 202.057 103.886) (end 196.469 103.886) (width 0.2) (layer "F.Cu") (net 32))
 (segment (start 189.677 97.094) (end 189.677 94.517999) (width 0.2) (layer "F.Cu") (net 32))
 (segment (start 203.454 99.441) (end 203.454 102.489) (width 0.2) (layer "F.Cu") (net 32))
 (segment (start 200.66 96.647) (end 203.454 99.441) (width 0.2) (layer "F.Cu") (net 32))
 (segment (start 203.454 102.489) (end 202.057 103.886) (width 0.2) (layer "F.Cu") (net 32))
 (segment (start 196.469 103.886) (end 189.677 97.094) (width 0.2) (layer "F.Cu") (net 32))
 (segment (start 191.515999 92.583) (end 190.627 92.583) (width 0.2) (layer "F.Cu") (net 16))
 (segment (start 200.66 101.727001) (end 191.515999 92.583) (width 0.2) (layer "F.Cu") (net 16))
 (segment (start 188.727 96.393) (end 188.727 94.62) (width 0.2) (layer "F.Cu") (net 10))
 (segment (start 188.727 94.62) (end 188.722 94.615) (width 0.2) (layer "F.Cu") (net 10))
 (segment (start 188.722 94.615) (end 184.848 94.615) (width 0.2) (layer "F.Cu") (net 10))
 (segment (start 166.575 88.914) (end 184.136 88.914) (width 0.2) (layer "F.Cu") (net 11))
 (segment (start 184.136 88.914) (end 185.634 87.416) (width 0.2) (layer "F.Cu") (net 11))
 (segment (start 185.634 87.416) (end 187.541 87.416) (width 0.2) (layer "F.Cu") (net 11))
 (segment (start 165.799 88.138) (end 166.575 88.914) (width 0.2) (layer "F.Cu") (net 11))
 (segment (start 187.063 89.416) (end 183.198 93.281) (width 0.2) (layer "F.Cu") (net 9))
 (segment (start 183.198 93.281) (end 183.198 94.615) (width 0.2) (layer "F.Cu") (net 9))
 (segment (start 187.541 89.416) (end 187.063 89.416) (width 0.2) (layer "F.Cu") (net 9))
 (segment (start 193.421 88.916) (end 193.421 91.186) (width 0.2) (layer "F.Cu") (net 13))
 (segment (start 183.388 90.678) (end 183.515 90.805) (width 0.2) (layer "F.Cu") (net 13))
 (segment (start 173.736 90.678) (end 183.388 90.678) (width 0.2) (layer "F.Cu") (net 13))
 (segment (start 173.736 92.583) (end 173.736 90.678) (width 0.2) (layer "F.Cu") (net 13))
 (segment (start 173.101 93.218) (end 173.736 92.583) (width 0.2) (layer "F.Cu") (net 13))
 (segment (start 173.926 94.043) (end 173.101 93.218) (width 0.2) (layer "F.Cu") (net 13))
 (segment (start 175.387 94.043) (end 173.926 94.043) (width 0.2) (layer "F.Cu") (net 13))
 (segment (start 191.516 88.916) (end 193.421 88.916) (width 0.2) (layer "F.Cu") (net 13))
 (via (at 193.421 91.186) (size 0.6) (drill 0.3) (layers "F.Cu" "B.Cu") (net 13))
 (via (at 183.515 90.805) (size 0.6) (drill 0.3) (layers "F.Cu" "B.Cu") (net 13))
 (segment (start 183.896 91.186) (end 193.421 91.186) (width 0.2) (layer "B.Cu") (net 13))
 (segment (start 183.515 90.805) (end 183.896 91.186) (width 0.2) (layer "B.Cu") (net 13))
 (segment (start 178.562 92.439064) (end 178.562 91.313) (width 0.2) (layer "F.Cu") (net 7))
 (segment (start 177.419 94.043) (end 177.419 93.582064) (width 0.2) (layer "F.Cu") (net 7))
 (segment (start 194.31 92.329) (end 194.31 88.416) (width 0.2) (layer "F.Cu") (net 7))
 (segment (start 177.419 93.582064) (end 178.562 92.439064) (width 0.2) (layer "F.Cu") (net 7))
 (segment (start 193.167 92.329) (end 194.31 92.329) (width 0.2) (layer "F.Cu") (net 7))
 (segment (start 194.31 88.416) (end 191.516 88.416) (width 0.2) (layer "F.Cu") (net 7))
 (via (at 178.562 91.313) (size 0.6) (drill 0.3) (layers "F.Cu" "B.Cu") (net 7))
 (via (at 193.167 92.329) (size 0.6) (drill 0.3) (layers "F.Cu" "B.Cu") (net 7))
 (segment (start 178.562 91.313) (end 183.134 91.313) (width 0.2) (layer "B.Cu") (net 7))
 (segment (start 184.15 92.329) (end 193.167 92.329) (width 0.2) (layer "B.Cu") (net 7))
 (segment (start 183.769 91.948) (end 184.15 92.329) (width 0.2) (layer "B.Cu") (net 7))
 (segment (start 183.134 91.313) (end 183.769 91.948) (width 0.2) (layer "B.Cu") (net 7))
 (segment (start 194.723 87.916) (end 191.516 87.916) (width 0.2) (layer "F.Cu") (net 17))
 (segment (start 193.167 93.345) (end 193.548 92.964) (width 0.2) (layer "F.Cu") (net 17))
 (segment (start 193.548 92.964) (end 194.818 92.964) (width 0.2) (layer "F.Cu") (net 17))
 (segment (start 194.818 92.964) (end 194.818 88.011) (width 0.2) (layer "F.Cu") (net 17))
 (segment (start 194.818 88.011) (end 194.723 87.916) (width 0.2) (layer "F.Cu") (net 17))
 (segment (start 180.023 94.043) (end 181.229 92.837) (width 0.2) (layer "F.Cu") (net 17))
 (segment (start 179.451 94.043) (end 180.023 94.043) (width 0.2) (layer "F.Cu") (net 17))
 (via (at 193.167 93.345) (size 0.6) (drill 0.3) (layers "F.Cu" "B.Cu") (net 17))
 (via (at 181.229 92.837) (size 0.6) (drill 0.3) (layers "F.Cu" "B.Cu") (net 17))
 (segment (start 181.229 92.837) (end 192.659 92.837) (width 0.2) (layer "B.Cu") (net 17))
 (segment (start 192.659 92.837) (end 193.167 93.345) (width 0.2) (layer "B.Cu") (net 17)))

